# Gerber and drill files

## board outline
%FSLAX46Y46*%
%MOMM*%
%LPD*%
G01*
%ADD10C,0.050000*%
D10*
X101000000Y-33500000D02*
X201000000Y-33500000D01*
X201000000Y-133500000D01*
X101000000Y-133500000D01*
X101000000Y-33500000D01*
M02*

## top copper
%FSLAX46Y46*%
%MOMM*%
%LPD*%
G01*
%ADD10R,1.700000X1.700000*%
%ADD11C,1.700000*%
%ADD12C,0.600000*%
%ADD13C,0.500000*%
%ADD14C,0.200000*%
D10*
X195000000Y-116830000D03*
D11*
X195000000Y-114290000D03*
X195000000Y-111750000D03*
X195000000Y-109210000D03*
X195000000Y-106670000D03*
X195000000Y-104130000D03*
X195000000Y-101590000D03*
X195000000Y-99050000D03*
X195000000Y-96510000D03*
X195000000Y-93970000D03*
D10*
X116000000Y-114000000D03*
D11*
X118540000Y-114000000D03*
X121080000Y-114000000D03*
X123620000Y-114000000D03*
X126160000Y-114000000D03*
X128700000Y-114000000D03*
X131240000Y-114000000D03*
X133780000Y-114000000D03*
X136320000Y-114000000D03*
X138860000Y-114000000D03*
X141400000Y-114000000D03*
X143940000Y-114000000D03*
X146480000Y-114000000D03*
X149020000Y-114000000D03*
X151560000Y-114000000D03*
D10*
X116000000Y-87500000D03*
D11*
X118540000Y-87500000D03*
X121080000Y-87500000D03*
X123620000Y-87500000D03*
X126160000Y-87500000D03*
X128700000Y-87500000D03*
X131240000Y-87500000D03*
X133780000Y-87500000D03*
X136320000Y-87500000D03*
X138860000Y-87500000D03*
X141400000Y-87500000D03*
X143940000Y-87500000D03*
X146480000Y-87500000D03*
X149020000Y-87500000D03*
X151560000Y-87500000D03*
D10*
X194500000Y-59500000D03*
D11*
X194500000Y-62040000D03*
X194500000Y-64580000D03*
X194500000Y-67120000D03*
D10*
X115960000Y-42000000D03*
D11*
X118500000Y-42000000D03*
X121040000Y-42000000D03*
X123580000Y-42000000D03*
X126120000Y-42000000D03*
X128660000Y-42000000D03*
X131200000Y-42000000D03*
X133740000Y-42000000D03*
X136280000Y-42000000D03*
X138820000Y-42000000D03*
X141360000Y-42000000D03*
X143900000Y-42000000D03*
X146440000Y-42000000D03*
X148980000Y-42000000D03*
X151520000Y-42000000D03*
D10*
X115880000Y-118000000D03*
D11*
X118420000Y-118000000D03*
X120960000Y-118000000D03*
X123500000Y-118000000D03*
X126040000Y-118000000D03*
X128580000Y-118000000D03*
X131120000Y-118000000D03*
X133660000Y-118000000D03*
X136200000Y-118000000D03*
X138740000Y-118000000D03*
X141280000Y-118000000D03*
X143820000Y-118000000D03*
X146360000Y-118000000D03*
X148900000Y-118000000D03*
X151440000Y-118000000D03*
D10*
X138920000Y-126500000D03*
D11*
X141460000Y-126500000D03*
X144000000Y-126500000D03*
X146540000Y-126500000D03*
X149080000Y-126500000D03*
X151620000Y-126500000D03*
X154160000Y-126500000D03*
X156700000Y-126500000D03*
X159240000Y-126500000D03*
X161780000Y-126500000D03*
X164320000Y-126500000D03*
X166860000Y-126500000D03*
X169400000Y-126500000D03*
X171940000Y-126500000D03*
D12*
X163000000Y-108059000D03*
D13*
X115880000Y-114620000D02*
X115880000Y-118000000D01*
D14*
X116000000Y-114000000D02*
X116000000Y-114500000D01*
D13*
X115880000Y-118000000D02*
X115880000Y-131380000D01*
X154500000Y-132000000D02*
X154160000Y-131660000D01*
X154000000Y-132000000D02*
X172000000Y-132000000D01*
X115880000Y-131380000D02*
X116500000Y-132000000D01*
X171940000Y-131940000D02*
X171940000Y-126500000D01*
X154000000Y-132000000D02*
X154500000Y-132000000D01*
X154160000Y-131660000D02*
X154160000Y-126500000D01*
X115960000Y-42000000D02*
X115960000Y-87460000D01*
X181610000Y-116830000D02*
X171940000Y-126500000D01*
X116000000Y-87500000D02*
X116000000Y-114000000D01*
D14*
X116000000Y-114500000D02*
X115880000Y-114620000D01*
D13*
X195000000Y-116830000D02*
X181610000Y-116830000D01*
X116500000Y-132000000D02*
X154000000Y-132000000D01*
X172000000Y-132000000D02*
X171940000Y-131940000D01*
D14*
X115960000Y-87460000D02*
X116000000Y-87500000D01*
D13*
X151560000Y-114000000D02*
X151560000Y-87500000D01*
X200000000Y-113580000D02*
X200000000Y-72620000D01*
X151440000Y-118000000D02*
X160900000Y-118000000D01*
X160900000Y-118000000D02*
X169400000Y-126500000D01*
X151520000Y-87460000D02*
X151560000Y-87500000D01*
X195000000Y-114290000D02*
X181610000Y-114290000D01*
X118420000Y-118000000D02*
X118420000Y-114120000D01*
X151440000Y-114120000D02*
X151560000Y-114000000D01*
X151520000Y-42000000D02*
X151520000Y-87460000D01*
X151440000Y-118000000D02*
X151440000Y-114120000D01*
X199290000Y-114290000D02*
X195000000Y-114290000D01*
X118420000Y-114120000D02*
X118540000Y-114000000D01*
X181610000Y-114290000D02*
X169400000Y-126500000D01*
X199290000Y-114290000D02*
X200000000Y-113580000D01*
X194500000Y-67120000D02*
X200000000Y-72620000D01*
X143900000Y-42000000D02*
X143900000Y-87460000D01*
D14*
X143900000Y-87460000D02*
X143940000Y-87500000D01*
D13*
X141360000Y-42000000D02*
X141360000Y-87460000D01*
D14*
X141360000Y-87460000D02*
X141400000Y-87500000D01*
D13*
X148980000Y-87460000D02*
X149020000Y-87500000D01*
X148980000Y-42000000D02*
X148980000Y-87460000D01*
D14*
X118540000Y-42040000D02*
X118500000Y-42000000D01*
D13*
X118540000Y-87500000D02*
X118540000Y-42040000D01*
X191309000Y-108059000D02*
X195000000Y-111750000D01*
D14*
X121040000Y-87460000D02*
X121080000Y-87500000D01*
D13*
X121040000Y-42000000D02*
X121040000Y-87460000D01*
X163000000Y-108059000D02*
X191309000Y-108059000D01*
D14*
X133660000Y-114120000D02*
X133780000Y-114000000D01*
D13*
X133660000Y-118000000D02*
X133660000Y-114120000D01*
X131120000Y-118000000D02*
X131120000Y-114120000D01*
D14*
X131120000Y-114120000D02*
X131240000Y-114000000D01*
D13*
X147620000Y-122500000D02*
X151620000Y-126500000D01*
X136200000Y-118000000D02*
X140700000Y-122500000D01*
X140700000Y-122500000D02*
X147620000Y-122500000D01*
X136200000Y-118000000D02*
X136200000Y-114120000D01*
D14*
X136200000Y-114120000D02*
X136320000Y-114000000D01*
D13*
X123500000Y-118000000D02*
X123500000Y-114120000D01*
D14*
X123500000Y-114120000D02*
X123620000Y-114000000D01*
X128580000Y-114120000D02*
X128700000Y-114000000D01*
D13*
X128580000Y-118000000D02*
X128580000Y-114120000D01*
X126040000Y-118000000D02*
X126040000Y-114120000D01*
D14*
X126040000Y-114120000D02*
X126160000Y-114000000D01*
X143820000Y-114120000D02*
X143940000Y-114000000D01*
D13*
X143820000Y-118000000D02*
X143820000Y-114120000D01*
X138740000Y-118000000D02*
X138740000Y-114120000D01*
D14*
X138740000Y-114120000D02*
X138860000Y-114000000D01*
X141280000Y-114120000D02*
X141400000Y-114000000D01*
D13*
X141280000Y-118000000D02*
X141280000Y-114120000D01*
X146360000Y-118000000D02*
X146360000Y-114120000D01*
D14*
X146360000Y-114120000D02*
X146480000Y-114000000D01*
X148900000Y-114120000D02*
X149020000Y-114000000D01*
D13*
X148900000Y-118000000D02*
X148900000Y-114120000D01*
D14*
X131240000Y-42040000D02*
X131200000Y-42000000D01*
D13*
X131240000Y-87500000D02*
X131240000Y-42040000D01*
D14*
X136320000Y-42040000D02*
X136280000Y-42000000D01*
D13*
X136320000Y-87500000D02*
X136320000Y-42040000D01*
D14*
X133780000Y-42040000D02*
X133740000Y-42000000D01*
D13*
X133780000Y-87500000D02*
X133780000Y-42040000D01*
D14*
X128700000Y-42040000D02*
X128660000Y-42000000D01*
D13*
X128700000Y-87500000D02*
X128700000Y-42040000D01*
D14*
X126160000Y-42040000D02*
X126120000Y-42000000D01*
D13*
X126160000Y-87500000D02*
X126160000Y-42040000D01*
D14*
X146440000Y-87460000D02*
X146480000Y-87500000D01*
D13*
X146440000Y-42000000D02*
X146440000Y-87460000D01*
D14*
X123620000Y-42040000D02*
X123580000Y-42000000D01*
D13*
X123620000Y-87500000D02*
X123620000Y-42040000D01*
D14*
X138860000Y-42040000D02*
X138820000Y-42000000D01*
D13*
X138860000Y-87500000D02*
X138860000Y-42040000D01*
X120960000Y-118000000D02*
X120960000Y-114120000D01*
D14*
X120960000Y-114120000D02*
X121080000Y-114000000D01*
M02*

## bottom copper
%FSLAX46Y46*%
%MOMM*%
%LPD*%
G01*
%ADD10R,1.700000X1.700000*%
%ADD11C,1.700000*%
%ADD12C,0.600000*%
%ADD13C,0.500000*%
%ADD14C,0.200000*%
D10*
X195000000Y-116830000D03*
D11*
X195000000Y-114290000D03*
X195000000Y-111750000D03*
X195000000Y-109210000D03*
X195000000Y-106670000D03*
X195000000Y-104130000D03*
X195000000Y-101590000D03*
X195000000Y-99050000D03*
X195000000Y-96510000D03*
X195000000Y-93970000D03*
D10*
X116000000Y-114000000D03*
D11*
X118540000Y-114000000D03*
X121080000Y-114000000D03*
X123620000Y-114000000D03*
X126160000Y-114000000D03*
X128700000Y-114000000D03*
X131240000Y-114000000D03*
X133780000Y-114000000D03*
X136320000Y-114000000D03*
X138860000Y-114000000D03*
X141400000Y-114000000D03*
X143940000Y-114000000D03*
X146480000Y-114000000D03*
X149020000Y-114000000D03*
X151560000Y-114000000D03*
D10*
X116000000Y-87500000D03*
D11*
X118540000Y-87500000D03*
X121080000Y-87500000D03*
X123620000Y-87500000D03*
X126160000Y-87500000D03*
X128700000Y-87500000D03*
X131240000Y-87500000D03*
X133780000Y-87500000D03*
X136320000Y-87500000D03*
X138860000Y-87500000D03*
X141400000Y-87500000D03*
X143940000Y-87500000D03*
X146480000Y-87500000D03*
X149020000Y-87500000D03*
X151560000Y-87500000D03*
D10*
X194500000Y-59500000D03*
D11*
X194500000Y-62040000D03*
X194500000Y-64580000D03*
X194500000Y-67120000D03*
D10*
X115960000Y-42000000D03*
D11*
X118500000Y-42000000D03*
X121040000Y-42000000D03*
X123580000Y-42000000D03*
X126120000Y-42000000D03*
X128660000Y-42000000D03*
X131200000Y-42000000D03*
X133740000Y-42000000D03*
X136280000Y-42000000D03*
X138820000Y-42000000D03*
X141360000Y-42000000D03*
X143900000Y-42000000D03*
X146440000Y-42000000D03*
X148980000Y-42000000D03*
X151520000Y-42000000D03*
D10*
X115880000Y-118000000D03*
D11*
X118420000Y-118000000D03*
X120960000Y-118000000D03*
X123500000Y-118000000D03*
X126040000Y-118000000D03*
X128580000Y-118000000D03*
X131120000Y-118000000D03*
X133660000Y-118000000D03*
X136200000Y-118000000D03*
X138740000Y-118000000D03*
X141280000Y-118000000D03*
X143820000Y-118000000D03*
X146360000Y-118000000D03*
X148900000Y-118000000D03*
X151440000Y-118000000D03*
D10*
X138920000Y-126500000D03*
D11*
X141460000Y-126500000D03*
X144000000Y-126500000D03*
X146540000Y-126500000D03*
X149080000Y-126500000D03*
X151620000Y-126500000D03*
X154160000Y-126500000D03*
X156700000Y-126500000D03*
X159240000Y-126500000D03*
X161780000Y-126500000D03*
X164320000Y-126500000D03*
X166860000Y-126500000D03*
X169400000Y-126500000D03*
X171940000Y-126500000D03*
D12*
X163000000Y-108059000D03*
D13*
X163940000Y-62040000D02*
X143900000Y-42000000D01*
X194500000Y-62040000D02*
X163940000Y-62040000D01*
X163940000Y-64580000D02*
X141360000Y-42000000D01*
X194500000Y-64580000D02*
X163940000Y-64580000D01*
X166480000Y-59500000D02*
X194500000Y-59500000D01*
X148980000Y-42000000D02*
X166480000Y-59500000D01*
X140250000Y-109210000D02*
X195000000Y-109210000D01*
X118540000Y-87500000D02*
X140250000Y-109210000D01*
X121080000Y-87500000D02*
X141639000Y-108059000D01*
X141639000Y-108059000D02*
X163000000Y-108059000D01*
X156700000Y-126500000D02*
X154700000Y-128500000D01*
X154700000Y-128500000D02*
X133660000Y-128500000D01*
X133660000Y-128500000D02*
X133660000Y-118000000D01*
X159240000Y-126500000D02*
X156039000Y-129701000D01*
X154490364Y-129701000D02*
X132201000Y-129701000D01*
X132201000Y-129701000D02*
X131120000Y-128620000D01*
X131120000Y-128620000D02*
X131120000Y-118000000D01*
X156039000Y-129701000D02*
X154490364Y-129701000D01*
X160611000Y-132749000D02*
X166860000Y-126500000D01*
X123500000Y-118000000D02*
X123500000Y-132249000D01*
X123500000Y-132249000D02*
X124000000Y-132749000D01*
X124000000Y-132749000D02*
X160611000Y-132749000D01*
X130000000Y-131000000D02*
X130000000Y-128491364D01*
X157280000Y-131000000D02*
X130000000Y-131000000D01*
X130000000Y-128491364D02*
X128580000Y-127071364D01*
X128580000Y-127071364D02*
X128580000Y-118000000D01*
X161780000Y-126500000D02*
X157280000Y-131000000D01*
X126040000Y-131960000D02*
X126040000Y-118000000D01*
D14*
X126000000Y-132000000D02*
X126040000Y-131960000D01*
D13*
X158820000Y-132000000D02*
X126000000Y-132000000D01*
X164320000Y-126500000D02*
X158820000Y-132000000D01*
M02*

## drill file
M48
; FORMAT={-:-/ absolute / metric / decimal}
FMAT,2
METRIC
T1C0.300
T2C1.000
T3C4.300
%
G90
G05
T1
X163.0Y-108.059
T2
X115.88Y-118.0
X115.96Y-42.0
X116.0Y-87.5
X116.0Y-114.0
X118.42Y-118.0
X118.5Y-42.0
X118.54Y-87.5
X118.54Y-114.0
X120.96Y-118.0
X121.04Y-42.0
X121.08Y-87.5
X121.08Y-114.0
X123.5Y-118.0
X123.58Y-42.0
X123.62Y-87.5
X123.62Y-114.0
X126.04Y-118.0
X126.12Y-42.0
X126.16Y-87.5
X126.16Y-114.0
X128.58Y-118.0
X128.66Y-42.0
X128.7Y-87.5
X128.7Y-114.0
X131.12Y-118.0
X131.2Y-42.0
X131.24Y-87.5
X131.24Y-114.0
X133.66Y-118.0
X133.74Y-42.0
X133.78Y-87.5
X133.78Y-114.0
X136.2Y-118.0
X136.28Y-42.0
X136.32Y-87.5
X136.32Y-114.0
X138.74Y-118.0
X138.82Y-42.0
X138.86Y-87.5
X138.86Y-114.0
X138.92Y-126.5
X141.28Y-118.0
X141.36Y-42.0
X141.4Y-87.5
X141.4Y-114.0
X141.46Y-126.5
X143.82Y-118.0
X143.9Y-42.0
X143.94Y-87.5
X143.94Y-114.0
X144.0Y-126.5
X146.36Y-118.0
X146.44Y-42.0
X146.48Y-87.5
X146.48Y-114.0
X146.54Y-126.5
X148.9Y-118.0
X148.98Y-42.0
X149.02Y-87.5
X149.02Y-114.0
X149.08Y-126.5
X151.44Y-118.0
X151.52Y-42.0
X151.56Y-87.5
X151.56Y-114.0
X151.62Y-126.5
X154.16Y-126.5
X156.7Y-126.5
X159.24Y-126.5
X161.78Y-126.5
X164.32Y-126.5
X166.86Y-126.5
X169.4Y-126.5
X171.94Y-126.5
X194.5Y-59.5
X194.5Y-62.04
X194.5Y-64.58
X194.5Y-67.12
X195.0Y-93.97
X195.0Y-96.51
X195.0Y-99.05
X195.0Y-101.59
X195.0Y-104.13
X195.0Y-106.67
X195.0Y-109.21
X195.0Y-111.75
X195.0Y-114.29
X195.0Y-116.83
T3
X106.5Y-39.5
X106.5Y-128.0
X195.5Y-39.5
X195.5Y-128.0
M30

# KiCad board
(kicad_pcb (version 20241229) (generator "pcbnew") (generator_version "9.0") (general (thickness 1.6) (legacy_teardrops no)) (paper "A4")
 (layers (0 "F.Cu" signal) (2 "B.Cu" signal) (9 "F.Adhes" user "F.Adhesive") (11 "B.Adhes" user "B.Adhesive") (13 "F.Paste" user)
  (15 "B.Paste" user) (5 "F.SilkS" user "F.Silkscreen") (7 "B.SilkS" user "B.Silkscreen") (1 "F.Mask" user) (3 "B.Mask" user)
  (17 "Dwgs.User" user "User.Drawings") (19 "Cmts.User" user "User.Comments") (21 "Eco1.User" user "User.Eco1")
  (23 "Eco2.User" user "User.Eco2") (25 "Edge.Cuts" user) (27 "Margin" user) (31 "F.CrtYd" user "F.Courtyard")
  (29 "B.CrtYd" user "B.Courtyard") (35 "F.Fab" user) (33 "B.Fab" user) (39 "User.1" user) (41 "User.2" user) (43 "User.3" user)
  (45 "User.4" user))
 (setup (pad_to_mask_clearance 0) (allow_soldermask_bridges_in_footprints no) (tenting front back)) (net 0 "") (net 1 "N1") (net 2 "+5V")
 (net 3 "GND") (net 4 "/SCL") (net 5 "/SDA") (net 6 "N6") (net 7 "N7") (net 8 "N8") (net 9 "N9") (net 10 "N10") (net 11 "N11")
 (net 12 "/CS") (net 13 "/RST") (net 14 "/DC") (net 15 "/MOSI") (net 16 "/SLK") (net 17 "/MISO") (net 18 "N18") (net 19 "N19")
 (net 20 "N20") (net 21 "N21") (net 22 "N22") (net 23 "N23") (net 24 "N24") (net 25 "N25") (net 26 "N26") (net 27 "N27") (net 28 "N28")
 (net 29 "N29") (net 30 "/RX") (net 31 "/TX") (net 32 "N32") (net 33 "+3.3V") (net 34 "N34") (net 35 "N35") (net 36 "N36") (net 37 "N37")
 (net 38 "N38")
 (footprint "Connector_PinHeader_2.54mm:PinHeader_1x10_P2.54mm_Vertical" (layer "F.Cu") (at 195 116.83 180)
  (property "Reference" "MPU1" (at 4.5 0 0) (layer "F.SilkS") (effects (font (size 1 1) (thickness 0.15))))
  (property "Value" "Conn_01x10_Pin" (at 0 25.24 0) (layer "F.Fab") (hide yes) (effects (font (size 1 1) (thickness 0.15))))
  (pad "1" thru_hole rect (at 0 0 180) (size 1.7 1.7) (drill 1) (layers "*.Cu" "*.Mask") (remove_unused_layers no) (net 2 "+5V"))
  (pad "2" thru_hole circle (at 0 2.54 180) (size 1.7 1.7) (drill 1) (layers "*.Cu" "*.Mask") (remove_unused_layers no) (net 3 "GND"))
  (pad "3" thru_hole circle (at 0 5.08 180) (size 1.7 1.7) (drill 1) (layers "*.Cu" "*.Mask") (remove_unused_layers no) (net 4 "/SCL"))
  (pad "4" thru_hole circle (at 0 7.62 180) (size 1.7 1.7) (drill 1) (layers "*.Cu" "*.Mask") (remove_unused_layers no) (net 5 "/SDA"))
  (pad "5" thru_hole circle (at 0 10.16 180) (size 1.7 1.7) (drill 1) (layers "*.Cu" "*.Mask") (remove_unused_layers no) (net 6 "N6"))
  (pad "6" thru_hole circle (at 0 12.7 180) (size 1.7 1.7) (drill 1) (layers "*.Cu" "*.Mask") (remove_unused_layers no) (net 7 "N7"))
  (pad "7" thru_hole circle (at 0 15.24 180) (size 1.7 1.7) (drill 1) (layers "*.Cu" "*.Mask") (remove_unused_layers no) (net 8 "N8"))
  (pad "8" thru_hole circle (at 0 17.78 180) (size 1.7 1.7) (drill 1) (layers "*.Cu" "*.Mask") (remove_unused_layers no) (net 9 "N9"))
  (pad "9" thru_hole circle (at 0 20.32 180) (size 1.7 1.7) (drill 1) (layers "*.Cu" "*.Mask") (remove_unused_layers no) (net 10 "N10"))
  (pad "10" thru_hole circle (at 0 22.86 180) (size 1.7 1.7) (drill 1) (layers "*.Cu" "*.Mask") (remove_unused_layers no) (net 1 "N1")))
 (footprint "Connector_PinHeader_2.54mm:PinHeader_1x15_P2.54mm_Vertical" (layer "F.Cu") (at 116 114 90)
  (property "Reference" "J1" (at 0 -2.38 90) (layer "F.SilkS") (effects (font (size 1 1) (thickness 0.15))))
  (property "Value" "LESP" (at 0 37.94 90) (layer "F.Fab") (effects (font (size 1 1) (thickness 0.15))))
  (pad "1" thru_hole rect (at 0 0 90) (size 1.7 1.7) (drill 1) (layers "*.Cu" "*.Mask") (remove_unused_layers no) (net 2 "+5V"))
  (pad "2" thru_hole circle (at 0 2.54 90) (size 1.7 1.7) (drill 1) (layers "*.Cu" "*.Mask") (remove_unused_layers no) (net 3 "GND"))
  (pad "3" thru_hole circle (at 0 5.08 90) (size 1.7 1.7) (drill 1) (layers "*.Cu" "*.Mask") (remove_unused_layers no) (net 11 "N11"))
  (pad "4" thru_hole circle (at 0 7.62 90) (size 1.7 1.7) (drill 1) (layers "*.Cu" "*.Mask") (remove_unused_layers no) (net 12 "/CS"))
  (pad "5" thru_hole circle (at 0 10.16 90) (size 1.7 1.7) (drill 1) (layers "*.Cu" "*.Mask") (remove_unused_layers no) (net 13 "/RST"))
  (pad "6" thru_hole circle (at 0 12.7 90) (size 1.7 1.7) (drill 1) (layers "*.Cu" "*.Mask") (remove_unused_layers no) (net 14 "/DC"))
  (pad "7" thru_hole circle (at 0 15.24 90) (size 1.7 1.7) (drill 1) (layers "*.Cu" "*.Mask") (remove_unused_layers no) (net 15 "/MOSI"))
  (pad "8" thru_hole circle (at 0 17.78 90) (size 1.7 1.7) (drill 1) (layers "*.Cu" "*.Mask") (remove_unused_layers no) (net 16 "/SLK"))
  (pad "9" thru_hole circle (at 0 20.32 90) (size 1.7 1.7) (drill 1) (layers "*.Cu" "*.Mask") (remove_unused_layers no) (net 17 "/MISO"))
  (pad "10" thru_hole circle (at 0 22.86 90) (size 1.7 1.7) (drill 1) (layers "*.Cu" "*.Mask") (remove_unused_layers no) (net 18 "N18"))
  (pad "11" thru_hole circle (at 0 25.4 90) (size 1.7 1.7) (drill 1) (layers "*.Cu" "*.Mask") (remove_unused_layers no) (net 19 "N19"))
  (pad "12" thru_hole circle (at 0 27.94 90) (size 1.7 1.7) (drill 1) (layers "*.Cu" "*.Mask") (remove_unused_layers no) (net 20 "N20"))
  (pad "13" thru_hole circle (at 0 30.48 90) (size 1.7 1.7) (drill 1) (layers "*.Cu" "*.Mask") (remove_unused_layers no) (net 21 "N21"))
  (pad "14" thru_hole circle (at 0 33.02 90) (size 1.7 1.7) (drill 1) (layers "*.Cu" "*.Mask") (remove_unused_layers no) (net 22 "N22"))
  (pad "15" thru_hole circle (at 0 35.56 90) (size 1.7 1.7) (drill 1) (layers "*.Cu" "*.Mask") (remove_unused_layers no) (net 3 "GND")))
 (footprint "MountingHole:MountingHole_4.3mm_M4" (layer "F.Cu") (at 106.5 128)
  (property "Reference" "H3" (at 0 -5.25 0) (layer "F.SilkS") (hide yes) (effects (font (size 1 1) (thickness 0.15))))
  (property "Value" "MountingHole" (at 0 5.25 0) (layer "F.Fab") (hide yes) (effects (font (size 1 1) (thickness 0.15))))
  (pad "" np_thru_hole circle (at 0 0) (size 4.3 4.3) (drill 4.3) (layers "*.Cu" "*.Mask")))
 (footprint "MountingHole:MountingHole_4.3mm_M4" (layer "F.Cu") (at 195.5 39.5)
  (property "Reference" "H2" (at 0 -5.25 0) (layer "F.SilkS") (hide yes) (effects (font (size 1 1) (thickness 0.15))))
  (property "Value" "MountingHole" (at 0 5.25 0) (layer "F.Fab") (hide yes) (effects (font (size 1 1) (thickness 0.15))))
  (pad "" np_thru_hole circle (at 0 0) (size 4.3 4.3) (drill 4.3) (layers "*.Cu" "*.Mask")))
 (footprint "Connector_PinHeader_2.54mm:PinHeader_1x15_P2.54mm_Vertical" (layer "F.Cu") (at 116 87.5 90)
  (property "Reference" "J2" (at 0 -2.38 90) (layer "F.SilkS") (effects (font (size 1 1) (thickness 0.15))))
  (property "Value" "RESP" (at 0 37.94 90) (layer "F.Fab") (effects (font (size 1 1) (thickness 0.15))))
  (pad "1" thru_hole rect (at 0 0 90) (size 1.7 1.7) (drill 1) (layers "*.Cu" "*.Mask") (remove_unused_layers no) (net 2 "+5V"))
  (pad "2" thru_hole circle (at 0 2.54 90) (size 1.7 1.7) (drill 1) (layers "*.Cu" "*.Mask") (remove_unused_layers no) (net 5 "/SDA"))
  (pad "3" thru_hole circle (at 0 5.08 90) (size 1.7 1.7) (drill 1) (layers "*.Cu" "*.Mask") (remove_unused_layers no) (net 4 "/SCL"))
  (pad "4" thru_hole circle (at 0 7.62 90) (size 1.7 1.7) (drill 1) (layers "*.Cu" "*.Mask") (remove_unused_layers no) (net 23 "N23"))
  (pad "5" thru_hole circle (at 0 10.16 90) (size 1.7 1.7) (drill 1) (layers "*.Cu" "*.Mask") (remove_unused_layers no) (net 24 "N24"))
  (pad "6" thru_hole circle (at 0 12.7 90) (size 1.7 1.7) (drill 1) (layers "*.Cu" "*.Mask") (remove_unused_layers no) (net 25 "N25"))
  (pad "7" thru_hole circle (at 0 15.24 90) (size 1.7 1.7) (drill 1) (layers "*.Cu" "*.Mask") (remove_unused_layers no) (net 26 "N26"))
  (pad "8" thru_hole circle (at 0 17.78 90) (size 1.7 1.7) (drill 1) (layers "*.Cu" "*.Mask") (remove_unused_layers no) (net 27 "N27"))
  (pad "9" thru_hole circle (at 0 20.32 90) (size 1.7 1.7) (drill 1) (layers "*.Cu" "*.Mask") (remove_unused_layers no) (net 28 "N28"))
  (pad "10" thru_hole circle (at 0 22.86 90) (size 1.7 1.7) (drill 1) (layers "*.Cu" "*.Mask") (remove_unused_layers no) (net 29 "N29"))
  (pad "11" thru_hole circle (at 0 25.4 90) (size 1.7 1.7) (drill 1) (layers "*.Cu" "*.Mask") (remove_unused_layers no) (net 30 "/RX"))
  (pad "12" thru_hole circle (at 0 27.94 90) (size 1.7 1.7) (drill 1) (layers "*.Cu" "*.Mask") (remove_unused_layers no) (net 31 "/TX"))
  (pad "13" thru_hole circle (at 0 30.48 90) (size 1.7 1.7) (drill 1) (layers "*.Cu" "*.Mask") (remove_unused_layers no) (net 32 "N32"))
  (pad "14" thru_hole circle (at 0 33.02 90) (size 1.7 1.7) (drill 1) (layers "*.Cu" "*.Mask") (remove_unused_layers no) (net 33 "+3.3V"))
  (pad "15" thru_hole circle (at 0 35.56 90) (size 1.7 1.7) (drill 1) (layers "*.Cu" "*.Mask") (remove_unused_layers no) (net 3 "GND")))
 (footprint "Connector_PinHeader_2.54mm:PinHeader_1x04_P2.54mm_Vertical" (layer "F.Cu") (at 194.5 59.5)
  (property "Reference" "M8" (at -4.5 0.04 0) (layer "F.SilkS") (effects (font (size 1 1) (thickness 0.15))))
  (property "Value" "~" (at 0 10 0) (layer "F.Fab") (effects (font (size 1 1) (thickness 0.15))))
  (pad "1" thru_hole rect (at 0 0) (size 1.7 1.7) (drill 1) (layers "*.Cu" "*.Mask") (remove_unused_layers no) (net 33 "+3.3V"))
  (pad "2" thru_hole circle (at 0 2.54) (size 1.7 1.7) (drill 1) (layers "*.Cu" "*.Mask") (remove_unused_layers no) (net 31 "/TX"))
  (pad "3" thru_hole circle (at 0 5.08) (size 1.7 1.7) (drill 1) (layers "*.Cu" "*.Mask") (remove_unused_layers no) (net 30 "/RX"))
  (pad "4" thru_hole circle (at 0 7.62) (size 1.7 1.7) (drill 1) (layers "*.Cu" "*.Mask") (remove_unused_layers no) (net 3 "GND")))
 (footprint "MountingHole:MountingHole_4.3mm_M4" (layer "F.Cu") (at 195.5 128)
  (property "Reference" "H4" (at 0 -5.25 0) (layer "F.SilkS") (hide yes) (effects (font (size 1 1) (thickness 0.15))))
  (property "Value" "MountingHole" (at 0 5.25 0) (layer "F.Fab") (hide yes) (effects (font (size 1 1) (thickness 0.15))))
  (pad "" np_thru_hole circle (at 0 0) (size 4.3 4.3) (drill 4.3) (layers "*.Cu" "*.Mask")))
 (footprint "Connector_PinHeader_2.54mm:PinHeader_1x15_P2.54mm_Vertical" (layer "F.Cu") (at 115.96 42 90)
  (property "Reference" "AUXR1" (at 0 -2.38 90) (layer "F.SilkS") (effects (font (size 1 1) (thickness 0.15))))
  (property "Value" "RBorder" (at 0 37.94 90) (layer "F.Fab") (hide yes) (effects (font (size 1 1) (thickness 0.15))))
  (pad "1" thru_hole rect (at 0 0 90) (size 1.7 1.7) (drill 1) (layers "*.Cu" "*.Mask") (remove_unused_layers no) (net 2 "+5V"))
  (pad "2" thru_hole circle (at 0 2.54 90) (size 1.7 1.7) (drill 1) (layers "*.Cu" "*.Mask") (remove_unused_layers no) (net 5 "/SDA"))
  (pad "3" thru_hole circle (at 0 5.08 90) (size 1.7 1.7) (drill 1) (layers "*.Cu" "*.Mask") (remove_unused_layers no) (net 4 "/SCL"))
  (pad "4" thru_hole circle (at 0 7.62 90) (size 1.7 1.7) (drill 1) (layers "*.Cu" "*.Mask") (remove_unused_layers no) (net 23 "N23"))
  (pad "5" thru_hole circle (at 0 10.16 90) (size 1.7 1.7) (drill 1) (layers "*.Cu" "*.Mask") (remove_unused_layers no) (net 24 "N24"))
  (pad "6" thru_hole circle (at 0 12.7 90) (size 1.7 1.7) (drill 1) (layers "*.Cu" "*.Mask") (remove_unused_layers no) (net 25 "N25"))
  (pad "7" thru_hole circle (at 0 15.24 90) (size 1.7 1.7) (drill 1) (layers "*.Cu" "*.Mask") (remove_unused_layers no) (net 26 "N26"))
  (pad "8" thru_hole circle (at 0 17.78 90) (size 1.7 1.7) (drill 1) (layers "*.Cu" "*.Mask") (remove_unused_layers no) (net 27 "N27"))
  (pad "9" thru_hole circle (at 0 20.32 90) (size 1.7 1.7) (drill 1) (layers "*.Cu" "*.Mask") (remove_unused_layers no) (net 28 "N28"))
  (pad "10" thru_hole circle (at 0 22.86 90) (size 1.7 1.7) (drill 1) (layers "*.Cu" "*.Mask") (remove_unused_layers no) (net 29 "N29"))
  (pad "11" thru_hole circle (at 0 25.4 90) (size 1.7 1.7) (drill 1) (layers "*.Cu" "*.Mask") (remove_unused_layers no) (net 30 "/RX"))
  (pad "12" thru_hole circle (at 0 27.94 90) (size 1.7 1.7) (drill 1) (layers "*.Cu" "*.Mask") (remove_unused_layers no) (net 31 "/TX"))
  (pad "13" thru_hole circle (at 0 30.48 90) (size 1.7 1.7) (drill 1) (layers "*.Cu" "*.Mask") (remove_unused_layers no) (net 32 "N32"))
  (pad "14" thru_hole circle (at 0 33.02 90) (size 1.7 1.7) (drill 1) (layers "*.Cu" "*.Mask") (remove_unused_layers no) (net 33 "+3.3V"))
  (pad "15" thru_hole circle (at 0 35.56 90) (size 1.7 1.7) (drill 1) (layers "*.Cu" "*.Mask") (remove_unused_layers no) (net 3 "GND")))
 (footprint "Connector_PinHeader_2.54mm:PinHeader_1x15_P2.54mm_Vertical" (layer "F.Cu") (at 115.88 118 90)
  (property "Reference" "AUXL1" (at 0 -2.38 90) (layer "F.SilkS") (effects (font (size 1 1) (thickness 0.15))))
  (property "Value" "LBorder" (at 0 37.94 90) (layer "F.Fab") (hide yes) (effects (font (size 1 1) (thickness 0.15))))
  (pad "1" thru_hole rect (at 0 0 90) (size 1.7 1.7) (drill 1) (layers "*.Cu" "*.Mask") (remove_unused_layers no) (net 2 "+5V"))
  (pad "2" thru_hole circle (at 0 2.54 90) (size 1.7 1.7) (drill 1) (layers "*.Cu" "*.Mask") (remove_unused_layers no) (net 3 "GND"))
  (pad "3" thru_hole circle (at 0 5.08 90) (size 1.7 1.7) (drill 1) (layers "*.Cu" "*.Mask") (remove_unused_layers no) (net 11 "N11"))
  (pad "4" thru_hole circle (at 0 7.62 90) (size 1.7 1.7) (drill 1) (layers "*.Cu" "*.Mask") (remove_unused_layers no) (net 12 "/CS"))
  (pad "5" thru_hole circle (at 0 10.16 90) (size 1.7 1.7) (drill 1) (layers "*.Cu" "*.Mask") (remove_unused_layers no) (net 13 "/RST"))
  (pad "6" thru_hole circle (at 0 12.7 90) (size 1.7 1.7) (drill 1) (layers "*.Cu" "*.Mask") (remove_unused_layers no) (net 14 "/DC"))
  (pad "7" thru_hole circle (at 0 15.24 90) (size 1.7 1.7) (drill 1) (layers "*.Cu" "*.Mask") (remove_unused_layers no) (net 15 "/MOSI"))
  (pad "8" thru_hole circle (at 0 17.78 90) (size 1.7 1.7) (drill 1) (layers "*.Cu" "*.Mask") (remove_unused_layers no) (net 16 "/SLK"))
  (pad "9" thru_hole circle (at 0 20.32 90) (size 1.7 1.7) (drill 1) (layers "*.Cu" "*.Mask") (remove_unused_layers no) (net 17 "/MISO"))
  (pad "10" thru_hole circle (at 0 22.86 90) (size 1.7 1.7) (drill 1) (layers "*.Cu" "*.Mask") (remove_unused_layers no) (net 18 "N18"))
  (pad "11" thru_hole circle (at 0 25.4 90) (size 1.7 1.7) (drill 1) (layers "*.Cu" "*.Mask") (remove_unused_layers no) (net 19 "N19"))
  (pad "12" thru_hole circle (at 0 27.94 90) (size 1.7 1.7) (drill 1) (layers "*.Cu" "*.Mask") (remove_unused_layers no) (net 20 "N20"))
  (pad "13" thru_hole circle (at 0 30.48 90) (size 1.7 1.7) (drill 1) (layers "*.Cu" "*.Mask") (remove_unused_layers no) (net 21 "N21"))
  (pad "14" thru_hole circle (at 0 33.02 90) (size 1.7 1.7) (drill 1) (layers "*.Cu" "*.Mask") (remove_unused_layers no) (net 22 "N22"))
  (pad "15" thru_hole circle (at 0 35.56 90) (size 1.7 1.7) (drill 1) (layers "*.Cu" "*.Mask") (remove_unused_layers no) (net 3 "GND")))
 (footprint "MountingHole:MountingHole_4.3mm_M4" (layer "F.Cu") (at 106.5 39.5)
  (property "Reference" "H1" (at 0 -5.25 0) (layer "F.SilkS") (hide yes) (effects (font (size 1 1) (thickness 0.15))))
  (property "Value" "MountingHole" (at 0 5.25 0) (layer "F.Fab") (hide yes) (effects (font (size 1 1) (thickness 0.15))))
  (pad "" np_thru_hole circle (at 0 0) (size 4.3 4.3) (drill 4.3) (layers "*.Cu" "*.Mask")))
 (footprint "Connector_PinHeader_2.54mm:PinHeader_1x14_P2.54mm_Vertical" (layer "B.Cu") (at 138.92 126.5 -90)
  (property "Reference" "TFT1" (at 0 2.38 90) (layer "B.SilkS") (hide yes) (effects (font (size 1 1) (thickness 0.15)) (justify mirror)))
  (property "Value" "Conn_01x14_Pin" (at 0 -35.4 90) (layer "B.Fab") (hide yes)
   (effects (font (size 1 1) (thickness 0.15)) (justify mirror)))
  (pad "1" thru_hole rect (at 0 0 270) (size 1.7 1.7) (drill 1) (layers "*.Cu" "*.Mask") (remove_unused_layers no) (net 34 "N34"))
  (pad "2" thru_hole circle (at 0 -2.54 270) (size 1.7 1.7) (drill 1) (layers "*.Cu" "*.Mask") (remove_unused_layers no) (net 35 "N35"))
  (pad "3" thru_hole circle (at 0 -5.08 270) (size 1.7 1.7) (drill 1) (layers "*.Cu" "*.Mask") (remove_unused_layers no) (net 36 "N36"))
  (pad "4" thru_hole circle (at 0 -7.62 270) (size 1.7 1.7) (drill 1) (layers "*.Cu" "*.Mask") (remove_unused_layers no) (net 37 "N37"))
  (pad "5" thru_hole circle (at 0 -10.16 270) (size 1.7 1.7) (drill 1) (layers "*.Cu" "*.Mask") (remove_unused_layers no) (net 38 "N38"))
  (pad "6" thru_hole circle (at 0 -12.7 270) (size 1.7 1.7) (drill 1) (layers "*.Cu" "*.Mask") (remove_unused_layers no) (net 17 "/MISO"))
  (pad "7" thru_hole circle (at 0 -15.24 270) (size 1.7 1.7) (drill 1) (layers "*.Cu" "*.Mask") (remove_unused_layers no) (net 2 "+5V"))
  (pad "8" thru_hole circle (at 0 -17.78 270) (size 1.7 1.7) (drill 1) (layers "*.Cu" "*.Mask") (remove_unused_layers no) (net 16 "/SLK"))
  (pad "9" thru_hole circle (at 0 -20.32 270) (size 1.7 1.7) (drill 1) (layers "*.Cu" "*.Mask") (remove_unused_layers no) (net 15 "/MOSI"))
  (pad "10" thru_hole circle (at 0 -22.86 270) (size 1.7 1.7) (drill 1) (layers "*.Cu" "*.Mask") (remove_unused_layers no) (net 14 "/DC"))
  (pad "11" thru_hole circle (at 0 -25.4 270) (size 1.7 1.7) (drill 1) (layers "*.Cu" "*.Mask") (remove_unused_layers no) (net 13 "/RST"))
  (pad "12" thru_hole circle (at 0 -27.94 270) (size 1.7 1.7) (drill 1) (layers "*.Cu" "*.Mask") (remove_unused_layers no) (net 12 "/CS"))
  (pad "13" thru_hole circle (at 0 -30.48 270) (size 1.7 1.7) (drill 1) (layers "*.Cu" "*.Mask") (remove_unused_layers no) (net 3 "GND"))
  (pad "14" thru_hole circle (at 0 -33.02 270) (size 1.7 1.7) (drill 1) (layers "*.Cu" "*.Mask") (remove_unused_layers no) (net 2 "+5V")))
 (gr_rect (start 101 33.5) (end 201 133.5) (stroke (width 0.05) (type default)) (fill no) (layer "Edge.Cuts"))
 (segment (start 115.88 114.62) (end 115.88 118) (width 0.5) (layer "F.Cu") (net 2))
 (segment (start 116 114) (end 116 114.5) (width 0.2) (layer "F.Cu") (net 2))
 (segment (start 115.88 118) (end 115.88 131.38) (width 0.5) (layer "F.Cu") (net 2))
 (segment (start 154.5 132) (end 154.16 131.66) (width 0.5) (layer "F.Cu") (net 2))
 (segment (start 154 132) (end 172 132) (width 0.5) (layer "F.Cu") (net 2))
 (segment (start 115.88 131.38) (end 116.5 132) (width 0.5) (layer "F.Cu") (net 2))
 (segment (start 171.94 131.94) (end 171.94 126.5) (width 0.5) (layer "F.Cu") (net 2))
 (segment (start 154 132) (end 154.5 132) (width 0.5) (layer "F.Cu") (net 2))
 (segment (start 154.16 131.66) (end 154.16 126.5) (width 0.5) (layer "F.Cu") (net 2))
 (segment (start 115.96 42) (end 115.96 87.46) (width 0.5) (layer "F.Cu") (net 2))
 (segment (start 181.61 116.83) (end 171.94 126.5) (width 0.5) (layer "F.Cu") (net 2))
 (segment (start 116 87.5) (end 116 114) (width 0.5) (layer "F.Cu") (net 2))
 (segment (start 116 114.5) (end 115.88 114.62) (width 0.2) (layer "F.Cu") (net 2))
 (segment (start 195 116.83) (end 181.61 116.83) (width 0.5) (layer "F.Cu") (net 2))
 (segment (start 116.5 132) (end 154 132) (width 0.5) (layer "F.Cu") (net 2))
 (segment (start 172 132) (end 171.94 131.94) (width 0.5) (layer "F.Cu") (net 2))
 (segment (start 115.96 87.46) (end 116 87.5) (width 0.2) (layer "F.Cu") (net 2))
 (segment (start 151.56 114) (end 151.56 87.5) (width 0.5) (layer "F.Cu") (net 3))
 (segment (start 200 113.58) (end 200 72.62) (width 0.5) (layer "F.Cu") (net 3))
 (segment (start 151.44 118) (end 160.9 118) (width 0.5) (layer "F.Cu") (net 3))
 (segment (start 160.9 118) (end 169.4 126.5) (width 0.5) (layer "F.Cu") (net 3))
 (segment (start 151.52 87.46) (end 151.56 87.5) (width 0.5) (layer "F.Cu") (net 3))
 (segment (start 195 114.29) (end 181.61 114.29) (width 0.5) (layer "F.Cu") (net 3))
 (segment (start 118.42 118) (end 118.42 114.12) (width 0.5) (layer "F.Cu") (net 3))
 (segment (start 151.44 114.12) (end 151.56 114) (width 0.5) (layer "F.Cu") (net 3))
 (segment (start 151.52 42) (end 151.52 87.46) (width 0.5) (layer "F.Cu") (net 3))
 (segment (start 151.44 118) (end 151.44 114.12) (width 0.5) (layer "F.Cu") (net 3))
 (segment (start 199.29 114.29) (end 195 114.29) (width 0.5) (layer "F.Cu") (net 3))
 (segment (start 118.42 114.12) (end 118.54 114) (width 0.5) (layer "F.Cu") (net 3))
 (segment (start 181.61 114.29) (end 169.4 126.5) (width 0.5) (layer "F.Cu") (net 3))
 (segment (start 199.29 114.29) (end 200 113.58) (width 0.5) (layer "F.Cu") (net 3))
 (segment (start 194.5 67.12) (end 200 72.62) (width 0.5) (layer "F.Cu") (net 3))
 (segment (start 143.9 42) (end 143.9 87.46) (width 0.5) (layer "F.Cu") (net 31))
 (segment (start 143.9 87.46) (end 143.94 87.5) (width 0.2) (layer "F.Cu") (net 31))
 (segment (start 163.94 62.04) (end 143.9 42) (width 0.5) (layer "B.Cu") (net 31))
 (segment (start 194.5 62.04) (end 163.94 62.04) (width 0.5) (layer "B.Cu") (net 31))
 (segment (start 141.36 42) (end 141.36 87.46) (width 0.5) (layer "F.Cu") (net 30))
 (segment (start 141.36 87.46) (end 141.4 87.5) (width 0.2) (layer "F.Cu") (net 30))
 (segment (start 163.94 64.58) (end 141.36 42) (width 0.5) (layer "B.Cu") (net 30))
 (segment (start 194.5 64.58) (end 163.94 64.58) (width 0.5) (layer "B.Cu") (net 30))
 (segment (start 148.98 87.46) (end 149.02 87.5) (width 0.5) (layer "F.Cu") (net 33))
 (segment (start 148.98 42) (end 148.98 87.46) (width 0.5) (layer "F.Cu") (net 33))
 (segment (start 166.48 59.5) (end 194.5 59.5) (width 0.5) (layer "B.Cu") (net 33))
 (segment (start 148.98 42) (end 166.48 59.5) (width 0.5) (layer "B.Cu") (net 33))
 (segment (start 118.54 42.04) (end 118.5 42) (width 0.2) (layer "F.Cu") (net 5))
 (segment (start 118.54 87.5) (end 118.54 42.04) (width 0.5) (layer "F.Cu") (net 5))
 (segment (start 140.25 109.21) (end 195 109.21) (width 0.5) (layer "B.Cu") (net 5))
 (segment (start 118.54 87.5) (end 140.25 109.21) (width 0.5) (layer "B.Cu") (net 5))
 (segment (start 191.309 108.059) (end 195 111.75) (width 0.5) (layer "F.Cu") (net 4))
 (segment (start 121.04 87.46) (end 121.08 87.5) (width 0.2) (layer "F.Cu") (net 4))
 (segment (start 121.04 42) (end 121.04 87.46) (width 0.5) (layer "F.Cu") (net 4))
 (segment (start 163 108.059) (end 191.309 108.059) (width 0.5) (layer "F.Cu") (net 4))
 (via (at 163 108.059) (size 0.6) (drill 0.3) (layers "F.Cu" "B.Cu") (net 4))
 (segment (start 121.08 87.5) (end 141.639 108.059) (width 0.5) (layer "B.Cu") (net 4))
 (segment (start 141.639 108.059) (end 163 108.059) (width 0.5) (layer "B.Cu") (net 4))
 (segment (start 133.66 114.12) (end 133.78 114) (width 0.2) (layer "F.Cu") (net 16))
 (segment (start 133.66 118) (end 133.66 114.12) (width 0.5) (layer "F.Cu") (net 16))
 (segment (start 156.7 126.5) (end 154.7 128.5) (width 0.5) (layer "B.Cu") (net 16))
 (segment (start 154.7 128.5) (end 133.66 128.5) (width 0.5) (layer "B.Cu") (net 16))
 (segment (start 133.66 128.5) (end 133.66 118) (width 0.5) (layer "B.Cu") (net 16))
 (segment (start 131.12 118) (end 131.12 114.12) (width 0.5) (layer "F.Cu") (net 15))
 (segment (start 131.12 114.12) (end 131.24 114) (width 0.2) (layer "F.Cu") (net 15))
 (segment (start 159.24 126.5) (end 156.039 129.701) (width 0.5) (layer "B.Cu") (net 15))
 (segment (start 154.490364 129.701) (end 132.201 129.701) (width 0.5) (layer "B.Cu") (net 15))
 (segment (start 132.201 129.701) (end 131.12 128.62) (width 0.5) (layer "B.Cu") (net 15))
 (segment (start 131.12 128.62) (end 131.12 118) (width 0.5) (layer "B.Cu") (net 15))
 (segment (start 156.039 129.701) (end 154.490364 129.701) (width 0.5) (layer "B.Cu") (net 15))
 (segment (start 147.62 122.5) (end 151.62 126.5) (width 0.5) (layer "F.Cu") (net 17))
 (segment (start 136.2 118) (end 140.7 122.5) (width 0.5) (layer "F.Cu") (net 17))
 (segment (start 140.7 122.5) (end 147.62 122.5) (width 0.5) (layer "F.Cu") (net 17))
 (segment (start 136.2 118) (end 136.2 114.12) (width 0.5) (layer "F.Cu") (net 17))
 (segment (start 136.2 114.12) (end 136.32 114) (width 0.2) (layer "F.Cu") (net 17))
 (segment (start 123.5 118) (end 123.5 114.12) (width 0.5) (layer "F.Cu") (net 12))
 (segment (start 123.5 114.12) (end 123.62 114) (width 0.2) (layer "F.Cu") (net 12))
 (segment (start 160.611 132.749) (end 166.86 126.5) (width 0.5) (layer "B.Cu") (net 12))
 (segment (start 123.5 118) (end 123.5 132.249) (width 0.5) (layer "B.Cu") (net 12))
 (segment (start 123.5 132.249) (end 124 132.749) (width 0.5) (layer "B.Cu") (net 12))
 (segment (start 124 132.749) (end 160.611 132.749) (width 0.5) (layer "B.Cu") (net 12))
 (segment (start 128.58 114.12) (end 128.7 114) (width 0.2) (layer "F.Cu") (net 14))
 (segment (start 128.58 118) (end 128.58 114.12) (width 0.5) (layer "F.Cu") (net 14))
 (segment (start 130 131) (end 130 128.491364) (width 0.5) (layer "B.Cu") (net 14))
 (segment (start 157.28 131) (end 130 131) (width 0.5) (layer "B.Cu") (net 14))
 (segment (start 130 128.491364) (end 128.58 127.071364) (width 0.5) (layer "B.Cu") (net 14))
 (segment (start 128.58 127.071364) (end 128.58 118) (width 0.5) (layer "B.Cu") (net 14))
 (segment (start 161.78 126.5) (end 157.28 131) (width 0.5) (layer "B.Cu") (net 14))
 (segment (start 126.04 118) (end 126.04 114.12) (width 0.5) (layer "F.Cu") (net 13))
 (segment (start 126.04 114.12) (end 126.16 114) (width 0.2) (layer "F.Cu") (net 13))
 (segment (start 126.04 131.96) (end 126.04 118) (width 0.5) (layer "B.Cu") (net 13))
 (segment (start 126 132) (end 126.04 131.96) (width 0.2) (layer "B.Cu") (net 13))
 (segment (start 158.82 132) (end 126 132) (width 0.5) (layer "B.Cu") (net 13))
 (segment (start 164.32 126.5) (end 158.82 132) (width 0.5) (layer "B.Cu") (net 13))
 (segment (start 143.82 114.12) (end 143.94 114) (width 0.2) (layer "F.Cu") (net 20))
 (segment (start 143.82 118) (end 143.82 114.12) (width 0.5) (layer "F.Cu") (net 20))
 (segment (start 138.74 118) (end 138.74 114.12) (width 0.5) (layer "F.Cu") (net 18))
 (segment (start 138.74 114.12) (end 138.86 114) (width 0.2) (layer "F.Cu") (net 18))
 (segment (start 141.28 114.12) (end 141.4 114) (width 0.2) (layer "F.Cu") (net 19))
 (segment (start 141.28 118) (end 141.28 114.12) (width 0.5) (layer "F.Cu") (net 19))
 (segment (start 146.36 118) (end 146.36 114.12) (width 0.5) (layer "F.Cu") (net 21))
 (segment (start 146.36 114.12) (end 146.48 114) (width 0.2) (layer "F.Cu") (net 21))
 (segment (start 148.9 114.12) (end 149.02 114) (width 0.2) (layer "F.Cu") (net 22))
 (segment (start 148.9 118) (end 148.9 114.12) (width 0.5) (layer "F.Cu") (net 22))
 (segment (start 131.24 42.04) (end 131.2 42) (width 0.2) (layer "F.Cu") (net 26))
 (segment (start 131.24 87.5) (end 131.24 42.04) (width 0.5) (layer "F.Cu") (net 26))
 (segment (start 136.32 42.04) (end 136.28 42) (width 0.2) (layer "F.Cu") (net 28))
 (segment (start 136.32 87.5) (end 136.32 42.04) (width 0.5) (layer "F.Cu") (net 28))
 (segment (start 133.78 42.04) (end 133.74 42) (width 0.2) (layer "F.Cu") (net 27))
 (segment (start 133.78 87.5) (end 133.78 42.04) (width 0.5) (layer "F.Cu") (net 27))
 (segment (start 128.7 42.04) (end 128.66 42) (width 0.2) (layer "F.Cu") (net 25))
 (segment (start 128.7 87.5) (end 128.7 42.04) (width 0.5) (layer "F.Cu") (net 25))
 (segment (start 126.16 42.04) (end 126.12 42) (width 0.2) (layer "F.Cu") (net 24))
 (segment (start 126.16 87.5) (end 126.16 42.04) (width 0.5) (layer "F.Cu") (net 24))
 (segment (start 146.44 87.46) (end 146.48 87.5) (width 0.2) (layer "F.Cu") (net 32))
 (segment (start 146.44 42) (end 146.44 87.46) (width 0.5) (layer "F.Cu") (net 32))
 (segment (start 123.62 42.04) (end 123.58 42) (width 0.2) (layer "F.Cu") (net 23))
 (segment (start 123.62 87.5) (end 123.62 42.04) (width 0.5) (layer "F.Cu") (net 23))
 (segment (start 138.86 42.04) (end 138.82 42) (width 0.2) (layer "F.Cu") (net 29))
 (segment (start 138.86 87.5) (end 138.86 42.04) (width 0.5) (layer "F.Cu") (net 29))
 (segment (start 120.96 118) (end 120.96 114.12) (width 0.5) (layer "F.Cu") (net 11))
 (segment (start 120.96 114.12) (end 121.08 114) (width 0.2) (layer "F.Cu") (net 11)))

